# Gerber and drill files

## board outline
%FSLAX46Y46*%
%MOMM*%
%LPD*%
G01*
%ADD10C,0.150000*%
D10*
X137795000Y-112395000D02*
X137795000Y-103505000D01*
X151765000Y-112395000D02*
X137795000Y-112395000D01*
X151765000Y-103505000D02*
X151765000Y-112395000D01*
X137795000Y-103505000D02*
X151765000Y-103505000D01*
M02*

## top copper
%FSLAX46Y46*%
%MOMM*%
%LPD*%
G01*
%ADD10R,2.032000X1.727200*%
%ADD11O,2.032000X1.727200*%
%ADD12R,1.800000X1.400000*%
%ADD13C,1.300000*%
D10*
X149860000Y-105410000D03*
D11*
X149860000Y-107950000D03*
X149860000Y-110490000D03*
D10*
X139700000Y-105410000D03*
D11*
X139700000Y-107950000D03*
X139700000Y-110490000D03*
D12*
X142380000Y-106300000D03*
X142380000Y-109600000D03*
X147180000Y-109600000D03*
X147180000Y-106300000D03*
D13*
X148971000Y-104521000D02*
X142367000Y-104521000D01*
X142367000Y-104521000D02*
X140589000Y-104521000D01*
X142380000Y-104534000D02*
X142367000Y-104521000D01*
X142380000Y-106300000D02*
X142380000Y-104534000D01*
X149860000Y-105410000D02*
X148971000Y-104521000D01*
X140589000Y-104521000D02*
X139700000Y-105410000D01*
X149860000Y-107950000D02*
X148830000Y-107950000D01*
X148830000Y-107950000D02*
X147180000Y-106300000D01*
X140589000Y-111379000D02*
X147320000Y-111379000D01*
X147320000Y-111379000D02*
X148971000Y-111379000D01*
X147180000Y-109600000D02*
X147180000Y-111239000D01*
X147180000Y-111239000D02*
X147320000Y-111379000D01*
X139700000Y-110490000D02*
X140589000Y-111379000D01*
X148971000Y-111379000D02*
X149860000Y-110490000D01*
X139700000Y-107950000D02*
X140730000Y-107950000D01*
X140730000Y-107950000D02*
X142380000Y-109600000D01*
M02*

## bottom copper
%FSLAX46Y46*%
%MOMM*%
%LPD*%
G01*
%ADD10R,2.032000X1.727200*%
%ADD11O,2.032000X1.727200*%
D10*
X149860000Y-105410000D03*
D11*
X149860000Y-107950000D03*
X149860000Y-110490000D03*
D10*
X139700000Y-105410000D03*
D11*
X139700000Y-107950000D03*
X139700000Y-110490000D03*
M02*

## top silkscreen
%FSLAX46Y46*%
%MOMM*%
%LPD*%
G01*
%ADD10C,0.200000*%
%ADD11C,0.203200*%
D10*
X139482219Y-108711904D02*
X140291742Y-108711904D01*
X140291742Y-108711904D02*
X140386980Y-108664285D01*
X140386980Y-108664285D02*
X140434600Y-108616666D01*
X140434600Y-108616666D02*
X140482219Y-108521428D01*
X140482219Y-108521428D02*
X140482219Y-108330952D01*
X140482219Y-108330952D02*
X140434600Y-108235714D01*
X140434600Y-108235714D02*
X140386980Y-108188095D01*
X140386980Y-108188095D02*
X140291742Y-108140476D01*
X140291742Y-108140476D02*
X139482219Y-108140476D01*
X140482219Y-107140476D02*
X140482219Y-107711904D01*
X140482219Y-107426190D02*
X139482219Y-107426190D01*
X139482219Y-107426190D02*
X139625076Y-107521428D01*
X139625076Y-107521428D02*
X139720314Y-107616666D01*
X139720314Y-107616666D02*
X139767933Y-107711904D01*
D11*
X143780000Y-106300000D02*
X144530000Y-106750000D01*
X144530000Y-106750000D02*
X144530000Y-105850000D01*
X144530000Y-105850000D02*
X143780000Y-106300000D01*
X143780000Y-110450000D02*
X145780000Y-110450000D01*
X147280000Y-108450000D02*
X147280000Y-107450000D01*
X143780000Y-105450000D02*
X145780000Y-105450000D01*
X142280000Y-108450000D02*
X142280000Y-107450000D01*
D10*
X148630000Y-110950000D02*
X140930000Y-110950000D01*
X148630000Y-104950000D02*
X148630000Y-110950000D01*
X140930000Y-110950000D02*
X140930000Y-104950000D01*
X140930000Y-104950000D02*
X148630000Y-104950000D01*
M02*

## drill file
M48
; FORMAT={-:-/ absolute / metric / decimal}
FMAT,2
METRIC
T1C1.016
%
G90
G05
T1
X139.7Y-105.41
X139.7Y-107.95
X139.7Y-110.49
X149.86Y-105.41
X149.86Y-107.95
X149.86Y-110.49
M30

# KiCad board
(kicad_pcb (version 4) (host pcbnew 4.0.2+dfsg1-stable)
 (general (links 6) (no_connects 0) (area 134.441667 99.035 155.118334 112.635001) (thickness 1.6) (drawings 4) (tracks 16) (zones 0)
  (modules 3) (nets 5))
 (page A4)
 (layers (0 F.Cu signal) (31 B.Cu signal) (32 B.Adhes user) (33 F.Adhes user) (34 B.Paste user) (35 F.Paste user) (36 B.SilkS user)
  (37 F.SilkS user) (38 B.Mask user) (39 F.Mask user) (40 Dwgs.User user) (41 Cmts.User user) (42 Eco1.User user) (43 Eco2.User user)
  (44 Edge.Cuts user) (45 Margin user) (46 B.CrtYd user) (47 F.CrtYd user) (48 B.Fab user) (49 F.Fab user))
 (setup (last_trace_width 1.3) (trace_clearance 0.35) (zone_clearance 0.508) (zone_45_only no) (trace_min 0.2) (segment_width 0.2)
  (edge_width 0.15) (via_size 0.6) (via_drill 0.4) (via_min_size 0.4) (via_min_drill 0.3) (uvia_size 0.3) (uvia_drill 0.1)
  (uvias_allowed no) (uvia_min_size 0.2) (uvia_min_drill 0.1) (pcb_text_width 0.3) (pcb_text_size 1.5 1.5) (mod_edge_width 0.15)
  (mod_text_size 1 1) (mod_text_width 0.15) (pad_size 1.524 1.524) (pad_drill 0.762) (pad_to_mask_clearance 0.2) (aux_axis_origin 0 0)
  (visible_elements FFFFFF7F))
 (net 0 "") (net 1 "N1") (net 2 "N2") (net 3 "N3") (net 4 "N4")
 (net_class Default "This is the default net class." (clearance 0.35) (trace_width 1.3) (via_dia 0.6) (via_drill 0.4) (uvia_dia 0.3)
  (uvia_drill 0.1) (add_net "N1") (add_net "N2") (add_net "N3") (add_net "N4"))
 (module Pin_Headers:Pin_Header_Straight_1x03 (layer B.Cu) (at 149.86 105.41 180)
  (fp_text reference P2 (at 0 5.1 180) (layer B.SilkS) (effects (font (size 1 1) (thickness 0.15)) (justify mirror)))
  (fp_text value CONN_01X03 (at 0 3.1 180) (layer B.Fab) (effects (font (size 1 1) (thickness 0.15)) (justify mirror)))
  (pad 1 thru_hole rect (at 0 0 180) (size 2.032 1.7272) (drill 1.016) (layers *.Cu *.Mask B.SilkS) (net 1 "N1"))
  (pad 2 thru_hole oval (at 0 -2.54 180) (size 2.032 1.7272) (drill 1.016) (layers *.Cu *.Mask B.SilkS) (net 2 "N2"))
  (pad 3 thru_hole oval (at 0 -5.08 180) (size 2.032 1.7272) (drill 1.016) (layers *.Cu *.Mask B.SilkS) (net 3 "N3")))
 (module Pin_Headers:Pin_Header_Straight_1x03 (layer B.Cu) (at 139.7 105.41 180)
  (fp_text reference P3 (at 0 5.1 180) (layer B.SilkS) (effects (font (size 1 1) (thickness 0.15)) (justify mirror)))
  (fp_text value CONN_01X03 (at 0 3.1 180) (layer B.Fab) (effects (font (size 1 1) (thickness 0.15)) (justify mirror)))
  (pad 1 thru_hole rect (at 0 0 180) (size 2.032 1.7272) (drill 1.016) (layers *.Cu *.Mask B.SilkS) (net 1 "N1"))
  (pad 2 thru_hole oval (at 0 -2.54 180) (size 2.032 1.7272) (drill 1.016) (layers *.Cu *.Mask B.SilkS) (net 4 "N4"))
  (pad 3 thru_hole oval (at 0 -5.08 180) (size 2.032 1.7272) (drill 1.016) (layers *.Cu *.Mask B.SilkS) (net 3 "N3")))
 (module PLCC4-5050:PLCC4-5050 (layer F.Cu) (at 144.78 107.95 90)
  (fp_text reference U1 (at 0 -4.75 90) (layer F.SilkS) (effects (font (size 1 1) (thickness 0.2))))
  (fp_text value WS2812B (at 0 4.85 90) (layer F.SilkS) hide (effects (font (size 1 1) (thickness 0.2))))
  (fp_line (start 1.65 -1) (end 1.2 -0.25) (layer F.SilkS) (width 0.2032))
  (fp_line (start 1.2 -0.25) (end 2.1 -0.25) (layer F.SilkS) (width 0.2032))
  (fp_line (start 2.1 -0.25) (end 1.65 -1) (layer F.SilkS) (width 0.2032))
  (fp_line (start -2.5 -1) (end -2.5 1) (layer F.SilkS) (width 0.2032))
  (fp_line (start -0.5 2.5) (end 0.5 2.5) (layer F.SilkS) (width 0.2032))
  (fp_line (start 2.5 -1) (end 2.5 1) (layer F.SilkS) (width 0.2032))
  (fp_line (start -0.5 -2.5) (end 0.5 -2.5) (layer F.SilkS) (width 0.2032))
  (fp_line (start -3 3.85) (end -3 -3.85) (layer F.SilkS) (width 0.2))
  (fp_line (start 3 3.85) (end -3 3.85) (layer F.SilkS) (width 0.2))
  (fp_line (start -3 -3.85) (end 3 -3.85) (layer F.SilkS) (width 0.2))
  (fp_line (start 3 -3.85) (end 3 3.85) (layer F.SilkS) (width 0.2))
  (pad 1 smd rect (at 1.65 -2.4 90) (size 1.4 1.8) (layers F.Cu F.Paste F.Mask) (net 1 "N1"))
  (pad 2 smd rect (at -1.65 -2.4 90) (size 1.4 1.8) (layers F.Cu F.Paste F.Mask) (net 4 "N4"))
  (pad 3 smd rect (at -1.65 2.4 90) (size 1.4 1.8) (layers F.Cu F.Paste F.Mask) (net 3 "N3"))
  (pad 4 smd rect (at 1.65 2.4 90) (size 1.4 1.8) (layers F.Cu F.Paste F.Mask) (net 2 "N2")))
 (gr_line (start 137.795 112.395) (end 137.795 103.505) (layer Edge.Cuts) (width 0.15))
 (gr_line (start 151.765 112.395) (end 137.795 112.395) (layer Edge.Cuts) (width 0.15))
 (gr_line (start 151.765 103.505) (end 151.765 112.395) (layer Edge.Cuts) (width 0.15))
 (gr_line (start 137.795 103.505) (end 151.765 103.505) (layer Edge.Cuts) (width 0.15))
 (segment (start 148.971 104.521) (end 142.367 104.521) (width 1.3) (layer F.Cu) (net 1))
 (segment (start 142.367 104.521) (end 140.589 104.521) (width 1.3) (layer F.Cu) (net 1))
 (segment (start 142.38 104.534) (end 142.367 104.521) (width 1.3) (layer F.Cu) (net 1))
 (segment (start 142.38 106.3) (end 142.38 104.534) (width 1.3) (layer F.Cu) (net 1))
 (segment (start 149.86 105.41) (end 148.971 104.521) (width 1.3) (layer F.Cu) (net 1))
 (segment (start 140.589 104.521) (end 139.7 105.41) (width 1.3) (layer F.Cu) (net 1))
 (segment (start 149.86 107.95) (end 148.83 107.95) (width 1.3) (layer F.Cu) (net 2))
 (segment (start 148.83 107.95) (end 147.18 106.3) (width 1.3) (layer F.Cu) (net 2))
 (segment (start 140.589 111.379) (end 147.32 111.379) (width 1.3) (layer F.Cu) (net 3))
 (segment (start 147.32 111.379) (end 148.971 111.379) (width 1.3) (layer F.Cu) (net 3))
 (segment (start 147.18 109.6) (end 147.18 111.239) (width 1.3) (layer F.Cu) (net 3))
 (segment (start 147.18 111.239) (end 147.32 111.379) (width 1.3) (layer F.Cu) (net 3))
 (segment (start 139.7 110.49) (end 140.589 111.379) (width 1.3) (layer F.Cu) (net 3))
 (segment (start 148.971 111.379) (end 149.86 110.49) (width 1.3) (layer F.Cu) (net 3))
 (segment (start 139.7 107.95) (end 140.73 107.95) (width 1.3) (layer F.Cu) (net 4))
 (segment (start 140.73 107.95) (end 142.38 109.6) (width 1.3) (layer F.Cu) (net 4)))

